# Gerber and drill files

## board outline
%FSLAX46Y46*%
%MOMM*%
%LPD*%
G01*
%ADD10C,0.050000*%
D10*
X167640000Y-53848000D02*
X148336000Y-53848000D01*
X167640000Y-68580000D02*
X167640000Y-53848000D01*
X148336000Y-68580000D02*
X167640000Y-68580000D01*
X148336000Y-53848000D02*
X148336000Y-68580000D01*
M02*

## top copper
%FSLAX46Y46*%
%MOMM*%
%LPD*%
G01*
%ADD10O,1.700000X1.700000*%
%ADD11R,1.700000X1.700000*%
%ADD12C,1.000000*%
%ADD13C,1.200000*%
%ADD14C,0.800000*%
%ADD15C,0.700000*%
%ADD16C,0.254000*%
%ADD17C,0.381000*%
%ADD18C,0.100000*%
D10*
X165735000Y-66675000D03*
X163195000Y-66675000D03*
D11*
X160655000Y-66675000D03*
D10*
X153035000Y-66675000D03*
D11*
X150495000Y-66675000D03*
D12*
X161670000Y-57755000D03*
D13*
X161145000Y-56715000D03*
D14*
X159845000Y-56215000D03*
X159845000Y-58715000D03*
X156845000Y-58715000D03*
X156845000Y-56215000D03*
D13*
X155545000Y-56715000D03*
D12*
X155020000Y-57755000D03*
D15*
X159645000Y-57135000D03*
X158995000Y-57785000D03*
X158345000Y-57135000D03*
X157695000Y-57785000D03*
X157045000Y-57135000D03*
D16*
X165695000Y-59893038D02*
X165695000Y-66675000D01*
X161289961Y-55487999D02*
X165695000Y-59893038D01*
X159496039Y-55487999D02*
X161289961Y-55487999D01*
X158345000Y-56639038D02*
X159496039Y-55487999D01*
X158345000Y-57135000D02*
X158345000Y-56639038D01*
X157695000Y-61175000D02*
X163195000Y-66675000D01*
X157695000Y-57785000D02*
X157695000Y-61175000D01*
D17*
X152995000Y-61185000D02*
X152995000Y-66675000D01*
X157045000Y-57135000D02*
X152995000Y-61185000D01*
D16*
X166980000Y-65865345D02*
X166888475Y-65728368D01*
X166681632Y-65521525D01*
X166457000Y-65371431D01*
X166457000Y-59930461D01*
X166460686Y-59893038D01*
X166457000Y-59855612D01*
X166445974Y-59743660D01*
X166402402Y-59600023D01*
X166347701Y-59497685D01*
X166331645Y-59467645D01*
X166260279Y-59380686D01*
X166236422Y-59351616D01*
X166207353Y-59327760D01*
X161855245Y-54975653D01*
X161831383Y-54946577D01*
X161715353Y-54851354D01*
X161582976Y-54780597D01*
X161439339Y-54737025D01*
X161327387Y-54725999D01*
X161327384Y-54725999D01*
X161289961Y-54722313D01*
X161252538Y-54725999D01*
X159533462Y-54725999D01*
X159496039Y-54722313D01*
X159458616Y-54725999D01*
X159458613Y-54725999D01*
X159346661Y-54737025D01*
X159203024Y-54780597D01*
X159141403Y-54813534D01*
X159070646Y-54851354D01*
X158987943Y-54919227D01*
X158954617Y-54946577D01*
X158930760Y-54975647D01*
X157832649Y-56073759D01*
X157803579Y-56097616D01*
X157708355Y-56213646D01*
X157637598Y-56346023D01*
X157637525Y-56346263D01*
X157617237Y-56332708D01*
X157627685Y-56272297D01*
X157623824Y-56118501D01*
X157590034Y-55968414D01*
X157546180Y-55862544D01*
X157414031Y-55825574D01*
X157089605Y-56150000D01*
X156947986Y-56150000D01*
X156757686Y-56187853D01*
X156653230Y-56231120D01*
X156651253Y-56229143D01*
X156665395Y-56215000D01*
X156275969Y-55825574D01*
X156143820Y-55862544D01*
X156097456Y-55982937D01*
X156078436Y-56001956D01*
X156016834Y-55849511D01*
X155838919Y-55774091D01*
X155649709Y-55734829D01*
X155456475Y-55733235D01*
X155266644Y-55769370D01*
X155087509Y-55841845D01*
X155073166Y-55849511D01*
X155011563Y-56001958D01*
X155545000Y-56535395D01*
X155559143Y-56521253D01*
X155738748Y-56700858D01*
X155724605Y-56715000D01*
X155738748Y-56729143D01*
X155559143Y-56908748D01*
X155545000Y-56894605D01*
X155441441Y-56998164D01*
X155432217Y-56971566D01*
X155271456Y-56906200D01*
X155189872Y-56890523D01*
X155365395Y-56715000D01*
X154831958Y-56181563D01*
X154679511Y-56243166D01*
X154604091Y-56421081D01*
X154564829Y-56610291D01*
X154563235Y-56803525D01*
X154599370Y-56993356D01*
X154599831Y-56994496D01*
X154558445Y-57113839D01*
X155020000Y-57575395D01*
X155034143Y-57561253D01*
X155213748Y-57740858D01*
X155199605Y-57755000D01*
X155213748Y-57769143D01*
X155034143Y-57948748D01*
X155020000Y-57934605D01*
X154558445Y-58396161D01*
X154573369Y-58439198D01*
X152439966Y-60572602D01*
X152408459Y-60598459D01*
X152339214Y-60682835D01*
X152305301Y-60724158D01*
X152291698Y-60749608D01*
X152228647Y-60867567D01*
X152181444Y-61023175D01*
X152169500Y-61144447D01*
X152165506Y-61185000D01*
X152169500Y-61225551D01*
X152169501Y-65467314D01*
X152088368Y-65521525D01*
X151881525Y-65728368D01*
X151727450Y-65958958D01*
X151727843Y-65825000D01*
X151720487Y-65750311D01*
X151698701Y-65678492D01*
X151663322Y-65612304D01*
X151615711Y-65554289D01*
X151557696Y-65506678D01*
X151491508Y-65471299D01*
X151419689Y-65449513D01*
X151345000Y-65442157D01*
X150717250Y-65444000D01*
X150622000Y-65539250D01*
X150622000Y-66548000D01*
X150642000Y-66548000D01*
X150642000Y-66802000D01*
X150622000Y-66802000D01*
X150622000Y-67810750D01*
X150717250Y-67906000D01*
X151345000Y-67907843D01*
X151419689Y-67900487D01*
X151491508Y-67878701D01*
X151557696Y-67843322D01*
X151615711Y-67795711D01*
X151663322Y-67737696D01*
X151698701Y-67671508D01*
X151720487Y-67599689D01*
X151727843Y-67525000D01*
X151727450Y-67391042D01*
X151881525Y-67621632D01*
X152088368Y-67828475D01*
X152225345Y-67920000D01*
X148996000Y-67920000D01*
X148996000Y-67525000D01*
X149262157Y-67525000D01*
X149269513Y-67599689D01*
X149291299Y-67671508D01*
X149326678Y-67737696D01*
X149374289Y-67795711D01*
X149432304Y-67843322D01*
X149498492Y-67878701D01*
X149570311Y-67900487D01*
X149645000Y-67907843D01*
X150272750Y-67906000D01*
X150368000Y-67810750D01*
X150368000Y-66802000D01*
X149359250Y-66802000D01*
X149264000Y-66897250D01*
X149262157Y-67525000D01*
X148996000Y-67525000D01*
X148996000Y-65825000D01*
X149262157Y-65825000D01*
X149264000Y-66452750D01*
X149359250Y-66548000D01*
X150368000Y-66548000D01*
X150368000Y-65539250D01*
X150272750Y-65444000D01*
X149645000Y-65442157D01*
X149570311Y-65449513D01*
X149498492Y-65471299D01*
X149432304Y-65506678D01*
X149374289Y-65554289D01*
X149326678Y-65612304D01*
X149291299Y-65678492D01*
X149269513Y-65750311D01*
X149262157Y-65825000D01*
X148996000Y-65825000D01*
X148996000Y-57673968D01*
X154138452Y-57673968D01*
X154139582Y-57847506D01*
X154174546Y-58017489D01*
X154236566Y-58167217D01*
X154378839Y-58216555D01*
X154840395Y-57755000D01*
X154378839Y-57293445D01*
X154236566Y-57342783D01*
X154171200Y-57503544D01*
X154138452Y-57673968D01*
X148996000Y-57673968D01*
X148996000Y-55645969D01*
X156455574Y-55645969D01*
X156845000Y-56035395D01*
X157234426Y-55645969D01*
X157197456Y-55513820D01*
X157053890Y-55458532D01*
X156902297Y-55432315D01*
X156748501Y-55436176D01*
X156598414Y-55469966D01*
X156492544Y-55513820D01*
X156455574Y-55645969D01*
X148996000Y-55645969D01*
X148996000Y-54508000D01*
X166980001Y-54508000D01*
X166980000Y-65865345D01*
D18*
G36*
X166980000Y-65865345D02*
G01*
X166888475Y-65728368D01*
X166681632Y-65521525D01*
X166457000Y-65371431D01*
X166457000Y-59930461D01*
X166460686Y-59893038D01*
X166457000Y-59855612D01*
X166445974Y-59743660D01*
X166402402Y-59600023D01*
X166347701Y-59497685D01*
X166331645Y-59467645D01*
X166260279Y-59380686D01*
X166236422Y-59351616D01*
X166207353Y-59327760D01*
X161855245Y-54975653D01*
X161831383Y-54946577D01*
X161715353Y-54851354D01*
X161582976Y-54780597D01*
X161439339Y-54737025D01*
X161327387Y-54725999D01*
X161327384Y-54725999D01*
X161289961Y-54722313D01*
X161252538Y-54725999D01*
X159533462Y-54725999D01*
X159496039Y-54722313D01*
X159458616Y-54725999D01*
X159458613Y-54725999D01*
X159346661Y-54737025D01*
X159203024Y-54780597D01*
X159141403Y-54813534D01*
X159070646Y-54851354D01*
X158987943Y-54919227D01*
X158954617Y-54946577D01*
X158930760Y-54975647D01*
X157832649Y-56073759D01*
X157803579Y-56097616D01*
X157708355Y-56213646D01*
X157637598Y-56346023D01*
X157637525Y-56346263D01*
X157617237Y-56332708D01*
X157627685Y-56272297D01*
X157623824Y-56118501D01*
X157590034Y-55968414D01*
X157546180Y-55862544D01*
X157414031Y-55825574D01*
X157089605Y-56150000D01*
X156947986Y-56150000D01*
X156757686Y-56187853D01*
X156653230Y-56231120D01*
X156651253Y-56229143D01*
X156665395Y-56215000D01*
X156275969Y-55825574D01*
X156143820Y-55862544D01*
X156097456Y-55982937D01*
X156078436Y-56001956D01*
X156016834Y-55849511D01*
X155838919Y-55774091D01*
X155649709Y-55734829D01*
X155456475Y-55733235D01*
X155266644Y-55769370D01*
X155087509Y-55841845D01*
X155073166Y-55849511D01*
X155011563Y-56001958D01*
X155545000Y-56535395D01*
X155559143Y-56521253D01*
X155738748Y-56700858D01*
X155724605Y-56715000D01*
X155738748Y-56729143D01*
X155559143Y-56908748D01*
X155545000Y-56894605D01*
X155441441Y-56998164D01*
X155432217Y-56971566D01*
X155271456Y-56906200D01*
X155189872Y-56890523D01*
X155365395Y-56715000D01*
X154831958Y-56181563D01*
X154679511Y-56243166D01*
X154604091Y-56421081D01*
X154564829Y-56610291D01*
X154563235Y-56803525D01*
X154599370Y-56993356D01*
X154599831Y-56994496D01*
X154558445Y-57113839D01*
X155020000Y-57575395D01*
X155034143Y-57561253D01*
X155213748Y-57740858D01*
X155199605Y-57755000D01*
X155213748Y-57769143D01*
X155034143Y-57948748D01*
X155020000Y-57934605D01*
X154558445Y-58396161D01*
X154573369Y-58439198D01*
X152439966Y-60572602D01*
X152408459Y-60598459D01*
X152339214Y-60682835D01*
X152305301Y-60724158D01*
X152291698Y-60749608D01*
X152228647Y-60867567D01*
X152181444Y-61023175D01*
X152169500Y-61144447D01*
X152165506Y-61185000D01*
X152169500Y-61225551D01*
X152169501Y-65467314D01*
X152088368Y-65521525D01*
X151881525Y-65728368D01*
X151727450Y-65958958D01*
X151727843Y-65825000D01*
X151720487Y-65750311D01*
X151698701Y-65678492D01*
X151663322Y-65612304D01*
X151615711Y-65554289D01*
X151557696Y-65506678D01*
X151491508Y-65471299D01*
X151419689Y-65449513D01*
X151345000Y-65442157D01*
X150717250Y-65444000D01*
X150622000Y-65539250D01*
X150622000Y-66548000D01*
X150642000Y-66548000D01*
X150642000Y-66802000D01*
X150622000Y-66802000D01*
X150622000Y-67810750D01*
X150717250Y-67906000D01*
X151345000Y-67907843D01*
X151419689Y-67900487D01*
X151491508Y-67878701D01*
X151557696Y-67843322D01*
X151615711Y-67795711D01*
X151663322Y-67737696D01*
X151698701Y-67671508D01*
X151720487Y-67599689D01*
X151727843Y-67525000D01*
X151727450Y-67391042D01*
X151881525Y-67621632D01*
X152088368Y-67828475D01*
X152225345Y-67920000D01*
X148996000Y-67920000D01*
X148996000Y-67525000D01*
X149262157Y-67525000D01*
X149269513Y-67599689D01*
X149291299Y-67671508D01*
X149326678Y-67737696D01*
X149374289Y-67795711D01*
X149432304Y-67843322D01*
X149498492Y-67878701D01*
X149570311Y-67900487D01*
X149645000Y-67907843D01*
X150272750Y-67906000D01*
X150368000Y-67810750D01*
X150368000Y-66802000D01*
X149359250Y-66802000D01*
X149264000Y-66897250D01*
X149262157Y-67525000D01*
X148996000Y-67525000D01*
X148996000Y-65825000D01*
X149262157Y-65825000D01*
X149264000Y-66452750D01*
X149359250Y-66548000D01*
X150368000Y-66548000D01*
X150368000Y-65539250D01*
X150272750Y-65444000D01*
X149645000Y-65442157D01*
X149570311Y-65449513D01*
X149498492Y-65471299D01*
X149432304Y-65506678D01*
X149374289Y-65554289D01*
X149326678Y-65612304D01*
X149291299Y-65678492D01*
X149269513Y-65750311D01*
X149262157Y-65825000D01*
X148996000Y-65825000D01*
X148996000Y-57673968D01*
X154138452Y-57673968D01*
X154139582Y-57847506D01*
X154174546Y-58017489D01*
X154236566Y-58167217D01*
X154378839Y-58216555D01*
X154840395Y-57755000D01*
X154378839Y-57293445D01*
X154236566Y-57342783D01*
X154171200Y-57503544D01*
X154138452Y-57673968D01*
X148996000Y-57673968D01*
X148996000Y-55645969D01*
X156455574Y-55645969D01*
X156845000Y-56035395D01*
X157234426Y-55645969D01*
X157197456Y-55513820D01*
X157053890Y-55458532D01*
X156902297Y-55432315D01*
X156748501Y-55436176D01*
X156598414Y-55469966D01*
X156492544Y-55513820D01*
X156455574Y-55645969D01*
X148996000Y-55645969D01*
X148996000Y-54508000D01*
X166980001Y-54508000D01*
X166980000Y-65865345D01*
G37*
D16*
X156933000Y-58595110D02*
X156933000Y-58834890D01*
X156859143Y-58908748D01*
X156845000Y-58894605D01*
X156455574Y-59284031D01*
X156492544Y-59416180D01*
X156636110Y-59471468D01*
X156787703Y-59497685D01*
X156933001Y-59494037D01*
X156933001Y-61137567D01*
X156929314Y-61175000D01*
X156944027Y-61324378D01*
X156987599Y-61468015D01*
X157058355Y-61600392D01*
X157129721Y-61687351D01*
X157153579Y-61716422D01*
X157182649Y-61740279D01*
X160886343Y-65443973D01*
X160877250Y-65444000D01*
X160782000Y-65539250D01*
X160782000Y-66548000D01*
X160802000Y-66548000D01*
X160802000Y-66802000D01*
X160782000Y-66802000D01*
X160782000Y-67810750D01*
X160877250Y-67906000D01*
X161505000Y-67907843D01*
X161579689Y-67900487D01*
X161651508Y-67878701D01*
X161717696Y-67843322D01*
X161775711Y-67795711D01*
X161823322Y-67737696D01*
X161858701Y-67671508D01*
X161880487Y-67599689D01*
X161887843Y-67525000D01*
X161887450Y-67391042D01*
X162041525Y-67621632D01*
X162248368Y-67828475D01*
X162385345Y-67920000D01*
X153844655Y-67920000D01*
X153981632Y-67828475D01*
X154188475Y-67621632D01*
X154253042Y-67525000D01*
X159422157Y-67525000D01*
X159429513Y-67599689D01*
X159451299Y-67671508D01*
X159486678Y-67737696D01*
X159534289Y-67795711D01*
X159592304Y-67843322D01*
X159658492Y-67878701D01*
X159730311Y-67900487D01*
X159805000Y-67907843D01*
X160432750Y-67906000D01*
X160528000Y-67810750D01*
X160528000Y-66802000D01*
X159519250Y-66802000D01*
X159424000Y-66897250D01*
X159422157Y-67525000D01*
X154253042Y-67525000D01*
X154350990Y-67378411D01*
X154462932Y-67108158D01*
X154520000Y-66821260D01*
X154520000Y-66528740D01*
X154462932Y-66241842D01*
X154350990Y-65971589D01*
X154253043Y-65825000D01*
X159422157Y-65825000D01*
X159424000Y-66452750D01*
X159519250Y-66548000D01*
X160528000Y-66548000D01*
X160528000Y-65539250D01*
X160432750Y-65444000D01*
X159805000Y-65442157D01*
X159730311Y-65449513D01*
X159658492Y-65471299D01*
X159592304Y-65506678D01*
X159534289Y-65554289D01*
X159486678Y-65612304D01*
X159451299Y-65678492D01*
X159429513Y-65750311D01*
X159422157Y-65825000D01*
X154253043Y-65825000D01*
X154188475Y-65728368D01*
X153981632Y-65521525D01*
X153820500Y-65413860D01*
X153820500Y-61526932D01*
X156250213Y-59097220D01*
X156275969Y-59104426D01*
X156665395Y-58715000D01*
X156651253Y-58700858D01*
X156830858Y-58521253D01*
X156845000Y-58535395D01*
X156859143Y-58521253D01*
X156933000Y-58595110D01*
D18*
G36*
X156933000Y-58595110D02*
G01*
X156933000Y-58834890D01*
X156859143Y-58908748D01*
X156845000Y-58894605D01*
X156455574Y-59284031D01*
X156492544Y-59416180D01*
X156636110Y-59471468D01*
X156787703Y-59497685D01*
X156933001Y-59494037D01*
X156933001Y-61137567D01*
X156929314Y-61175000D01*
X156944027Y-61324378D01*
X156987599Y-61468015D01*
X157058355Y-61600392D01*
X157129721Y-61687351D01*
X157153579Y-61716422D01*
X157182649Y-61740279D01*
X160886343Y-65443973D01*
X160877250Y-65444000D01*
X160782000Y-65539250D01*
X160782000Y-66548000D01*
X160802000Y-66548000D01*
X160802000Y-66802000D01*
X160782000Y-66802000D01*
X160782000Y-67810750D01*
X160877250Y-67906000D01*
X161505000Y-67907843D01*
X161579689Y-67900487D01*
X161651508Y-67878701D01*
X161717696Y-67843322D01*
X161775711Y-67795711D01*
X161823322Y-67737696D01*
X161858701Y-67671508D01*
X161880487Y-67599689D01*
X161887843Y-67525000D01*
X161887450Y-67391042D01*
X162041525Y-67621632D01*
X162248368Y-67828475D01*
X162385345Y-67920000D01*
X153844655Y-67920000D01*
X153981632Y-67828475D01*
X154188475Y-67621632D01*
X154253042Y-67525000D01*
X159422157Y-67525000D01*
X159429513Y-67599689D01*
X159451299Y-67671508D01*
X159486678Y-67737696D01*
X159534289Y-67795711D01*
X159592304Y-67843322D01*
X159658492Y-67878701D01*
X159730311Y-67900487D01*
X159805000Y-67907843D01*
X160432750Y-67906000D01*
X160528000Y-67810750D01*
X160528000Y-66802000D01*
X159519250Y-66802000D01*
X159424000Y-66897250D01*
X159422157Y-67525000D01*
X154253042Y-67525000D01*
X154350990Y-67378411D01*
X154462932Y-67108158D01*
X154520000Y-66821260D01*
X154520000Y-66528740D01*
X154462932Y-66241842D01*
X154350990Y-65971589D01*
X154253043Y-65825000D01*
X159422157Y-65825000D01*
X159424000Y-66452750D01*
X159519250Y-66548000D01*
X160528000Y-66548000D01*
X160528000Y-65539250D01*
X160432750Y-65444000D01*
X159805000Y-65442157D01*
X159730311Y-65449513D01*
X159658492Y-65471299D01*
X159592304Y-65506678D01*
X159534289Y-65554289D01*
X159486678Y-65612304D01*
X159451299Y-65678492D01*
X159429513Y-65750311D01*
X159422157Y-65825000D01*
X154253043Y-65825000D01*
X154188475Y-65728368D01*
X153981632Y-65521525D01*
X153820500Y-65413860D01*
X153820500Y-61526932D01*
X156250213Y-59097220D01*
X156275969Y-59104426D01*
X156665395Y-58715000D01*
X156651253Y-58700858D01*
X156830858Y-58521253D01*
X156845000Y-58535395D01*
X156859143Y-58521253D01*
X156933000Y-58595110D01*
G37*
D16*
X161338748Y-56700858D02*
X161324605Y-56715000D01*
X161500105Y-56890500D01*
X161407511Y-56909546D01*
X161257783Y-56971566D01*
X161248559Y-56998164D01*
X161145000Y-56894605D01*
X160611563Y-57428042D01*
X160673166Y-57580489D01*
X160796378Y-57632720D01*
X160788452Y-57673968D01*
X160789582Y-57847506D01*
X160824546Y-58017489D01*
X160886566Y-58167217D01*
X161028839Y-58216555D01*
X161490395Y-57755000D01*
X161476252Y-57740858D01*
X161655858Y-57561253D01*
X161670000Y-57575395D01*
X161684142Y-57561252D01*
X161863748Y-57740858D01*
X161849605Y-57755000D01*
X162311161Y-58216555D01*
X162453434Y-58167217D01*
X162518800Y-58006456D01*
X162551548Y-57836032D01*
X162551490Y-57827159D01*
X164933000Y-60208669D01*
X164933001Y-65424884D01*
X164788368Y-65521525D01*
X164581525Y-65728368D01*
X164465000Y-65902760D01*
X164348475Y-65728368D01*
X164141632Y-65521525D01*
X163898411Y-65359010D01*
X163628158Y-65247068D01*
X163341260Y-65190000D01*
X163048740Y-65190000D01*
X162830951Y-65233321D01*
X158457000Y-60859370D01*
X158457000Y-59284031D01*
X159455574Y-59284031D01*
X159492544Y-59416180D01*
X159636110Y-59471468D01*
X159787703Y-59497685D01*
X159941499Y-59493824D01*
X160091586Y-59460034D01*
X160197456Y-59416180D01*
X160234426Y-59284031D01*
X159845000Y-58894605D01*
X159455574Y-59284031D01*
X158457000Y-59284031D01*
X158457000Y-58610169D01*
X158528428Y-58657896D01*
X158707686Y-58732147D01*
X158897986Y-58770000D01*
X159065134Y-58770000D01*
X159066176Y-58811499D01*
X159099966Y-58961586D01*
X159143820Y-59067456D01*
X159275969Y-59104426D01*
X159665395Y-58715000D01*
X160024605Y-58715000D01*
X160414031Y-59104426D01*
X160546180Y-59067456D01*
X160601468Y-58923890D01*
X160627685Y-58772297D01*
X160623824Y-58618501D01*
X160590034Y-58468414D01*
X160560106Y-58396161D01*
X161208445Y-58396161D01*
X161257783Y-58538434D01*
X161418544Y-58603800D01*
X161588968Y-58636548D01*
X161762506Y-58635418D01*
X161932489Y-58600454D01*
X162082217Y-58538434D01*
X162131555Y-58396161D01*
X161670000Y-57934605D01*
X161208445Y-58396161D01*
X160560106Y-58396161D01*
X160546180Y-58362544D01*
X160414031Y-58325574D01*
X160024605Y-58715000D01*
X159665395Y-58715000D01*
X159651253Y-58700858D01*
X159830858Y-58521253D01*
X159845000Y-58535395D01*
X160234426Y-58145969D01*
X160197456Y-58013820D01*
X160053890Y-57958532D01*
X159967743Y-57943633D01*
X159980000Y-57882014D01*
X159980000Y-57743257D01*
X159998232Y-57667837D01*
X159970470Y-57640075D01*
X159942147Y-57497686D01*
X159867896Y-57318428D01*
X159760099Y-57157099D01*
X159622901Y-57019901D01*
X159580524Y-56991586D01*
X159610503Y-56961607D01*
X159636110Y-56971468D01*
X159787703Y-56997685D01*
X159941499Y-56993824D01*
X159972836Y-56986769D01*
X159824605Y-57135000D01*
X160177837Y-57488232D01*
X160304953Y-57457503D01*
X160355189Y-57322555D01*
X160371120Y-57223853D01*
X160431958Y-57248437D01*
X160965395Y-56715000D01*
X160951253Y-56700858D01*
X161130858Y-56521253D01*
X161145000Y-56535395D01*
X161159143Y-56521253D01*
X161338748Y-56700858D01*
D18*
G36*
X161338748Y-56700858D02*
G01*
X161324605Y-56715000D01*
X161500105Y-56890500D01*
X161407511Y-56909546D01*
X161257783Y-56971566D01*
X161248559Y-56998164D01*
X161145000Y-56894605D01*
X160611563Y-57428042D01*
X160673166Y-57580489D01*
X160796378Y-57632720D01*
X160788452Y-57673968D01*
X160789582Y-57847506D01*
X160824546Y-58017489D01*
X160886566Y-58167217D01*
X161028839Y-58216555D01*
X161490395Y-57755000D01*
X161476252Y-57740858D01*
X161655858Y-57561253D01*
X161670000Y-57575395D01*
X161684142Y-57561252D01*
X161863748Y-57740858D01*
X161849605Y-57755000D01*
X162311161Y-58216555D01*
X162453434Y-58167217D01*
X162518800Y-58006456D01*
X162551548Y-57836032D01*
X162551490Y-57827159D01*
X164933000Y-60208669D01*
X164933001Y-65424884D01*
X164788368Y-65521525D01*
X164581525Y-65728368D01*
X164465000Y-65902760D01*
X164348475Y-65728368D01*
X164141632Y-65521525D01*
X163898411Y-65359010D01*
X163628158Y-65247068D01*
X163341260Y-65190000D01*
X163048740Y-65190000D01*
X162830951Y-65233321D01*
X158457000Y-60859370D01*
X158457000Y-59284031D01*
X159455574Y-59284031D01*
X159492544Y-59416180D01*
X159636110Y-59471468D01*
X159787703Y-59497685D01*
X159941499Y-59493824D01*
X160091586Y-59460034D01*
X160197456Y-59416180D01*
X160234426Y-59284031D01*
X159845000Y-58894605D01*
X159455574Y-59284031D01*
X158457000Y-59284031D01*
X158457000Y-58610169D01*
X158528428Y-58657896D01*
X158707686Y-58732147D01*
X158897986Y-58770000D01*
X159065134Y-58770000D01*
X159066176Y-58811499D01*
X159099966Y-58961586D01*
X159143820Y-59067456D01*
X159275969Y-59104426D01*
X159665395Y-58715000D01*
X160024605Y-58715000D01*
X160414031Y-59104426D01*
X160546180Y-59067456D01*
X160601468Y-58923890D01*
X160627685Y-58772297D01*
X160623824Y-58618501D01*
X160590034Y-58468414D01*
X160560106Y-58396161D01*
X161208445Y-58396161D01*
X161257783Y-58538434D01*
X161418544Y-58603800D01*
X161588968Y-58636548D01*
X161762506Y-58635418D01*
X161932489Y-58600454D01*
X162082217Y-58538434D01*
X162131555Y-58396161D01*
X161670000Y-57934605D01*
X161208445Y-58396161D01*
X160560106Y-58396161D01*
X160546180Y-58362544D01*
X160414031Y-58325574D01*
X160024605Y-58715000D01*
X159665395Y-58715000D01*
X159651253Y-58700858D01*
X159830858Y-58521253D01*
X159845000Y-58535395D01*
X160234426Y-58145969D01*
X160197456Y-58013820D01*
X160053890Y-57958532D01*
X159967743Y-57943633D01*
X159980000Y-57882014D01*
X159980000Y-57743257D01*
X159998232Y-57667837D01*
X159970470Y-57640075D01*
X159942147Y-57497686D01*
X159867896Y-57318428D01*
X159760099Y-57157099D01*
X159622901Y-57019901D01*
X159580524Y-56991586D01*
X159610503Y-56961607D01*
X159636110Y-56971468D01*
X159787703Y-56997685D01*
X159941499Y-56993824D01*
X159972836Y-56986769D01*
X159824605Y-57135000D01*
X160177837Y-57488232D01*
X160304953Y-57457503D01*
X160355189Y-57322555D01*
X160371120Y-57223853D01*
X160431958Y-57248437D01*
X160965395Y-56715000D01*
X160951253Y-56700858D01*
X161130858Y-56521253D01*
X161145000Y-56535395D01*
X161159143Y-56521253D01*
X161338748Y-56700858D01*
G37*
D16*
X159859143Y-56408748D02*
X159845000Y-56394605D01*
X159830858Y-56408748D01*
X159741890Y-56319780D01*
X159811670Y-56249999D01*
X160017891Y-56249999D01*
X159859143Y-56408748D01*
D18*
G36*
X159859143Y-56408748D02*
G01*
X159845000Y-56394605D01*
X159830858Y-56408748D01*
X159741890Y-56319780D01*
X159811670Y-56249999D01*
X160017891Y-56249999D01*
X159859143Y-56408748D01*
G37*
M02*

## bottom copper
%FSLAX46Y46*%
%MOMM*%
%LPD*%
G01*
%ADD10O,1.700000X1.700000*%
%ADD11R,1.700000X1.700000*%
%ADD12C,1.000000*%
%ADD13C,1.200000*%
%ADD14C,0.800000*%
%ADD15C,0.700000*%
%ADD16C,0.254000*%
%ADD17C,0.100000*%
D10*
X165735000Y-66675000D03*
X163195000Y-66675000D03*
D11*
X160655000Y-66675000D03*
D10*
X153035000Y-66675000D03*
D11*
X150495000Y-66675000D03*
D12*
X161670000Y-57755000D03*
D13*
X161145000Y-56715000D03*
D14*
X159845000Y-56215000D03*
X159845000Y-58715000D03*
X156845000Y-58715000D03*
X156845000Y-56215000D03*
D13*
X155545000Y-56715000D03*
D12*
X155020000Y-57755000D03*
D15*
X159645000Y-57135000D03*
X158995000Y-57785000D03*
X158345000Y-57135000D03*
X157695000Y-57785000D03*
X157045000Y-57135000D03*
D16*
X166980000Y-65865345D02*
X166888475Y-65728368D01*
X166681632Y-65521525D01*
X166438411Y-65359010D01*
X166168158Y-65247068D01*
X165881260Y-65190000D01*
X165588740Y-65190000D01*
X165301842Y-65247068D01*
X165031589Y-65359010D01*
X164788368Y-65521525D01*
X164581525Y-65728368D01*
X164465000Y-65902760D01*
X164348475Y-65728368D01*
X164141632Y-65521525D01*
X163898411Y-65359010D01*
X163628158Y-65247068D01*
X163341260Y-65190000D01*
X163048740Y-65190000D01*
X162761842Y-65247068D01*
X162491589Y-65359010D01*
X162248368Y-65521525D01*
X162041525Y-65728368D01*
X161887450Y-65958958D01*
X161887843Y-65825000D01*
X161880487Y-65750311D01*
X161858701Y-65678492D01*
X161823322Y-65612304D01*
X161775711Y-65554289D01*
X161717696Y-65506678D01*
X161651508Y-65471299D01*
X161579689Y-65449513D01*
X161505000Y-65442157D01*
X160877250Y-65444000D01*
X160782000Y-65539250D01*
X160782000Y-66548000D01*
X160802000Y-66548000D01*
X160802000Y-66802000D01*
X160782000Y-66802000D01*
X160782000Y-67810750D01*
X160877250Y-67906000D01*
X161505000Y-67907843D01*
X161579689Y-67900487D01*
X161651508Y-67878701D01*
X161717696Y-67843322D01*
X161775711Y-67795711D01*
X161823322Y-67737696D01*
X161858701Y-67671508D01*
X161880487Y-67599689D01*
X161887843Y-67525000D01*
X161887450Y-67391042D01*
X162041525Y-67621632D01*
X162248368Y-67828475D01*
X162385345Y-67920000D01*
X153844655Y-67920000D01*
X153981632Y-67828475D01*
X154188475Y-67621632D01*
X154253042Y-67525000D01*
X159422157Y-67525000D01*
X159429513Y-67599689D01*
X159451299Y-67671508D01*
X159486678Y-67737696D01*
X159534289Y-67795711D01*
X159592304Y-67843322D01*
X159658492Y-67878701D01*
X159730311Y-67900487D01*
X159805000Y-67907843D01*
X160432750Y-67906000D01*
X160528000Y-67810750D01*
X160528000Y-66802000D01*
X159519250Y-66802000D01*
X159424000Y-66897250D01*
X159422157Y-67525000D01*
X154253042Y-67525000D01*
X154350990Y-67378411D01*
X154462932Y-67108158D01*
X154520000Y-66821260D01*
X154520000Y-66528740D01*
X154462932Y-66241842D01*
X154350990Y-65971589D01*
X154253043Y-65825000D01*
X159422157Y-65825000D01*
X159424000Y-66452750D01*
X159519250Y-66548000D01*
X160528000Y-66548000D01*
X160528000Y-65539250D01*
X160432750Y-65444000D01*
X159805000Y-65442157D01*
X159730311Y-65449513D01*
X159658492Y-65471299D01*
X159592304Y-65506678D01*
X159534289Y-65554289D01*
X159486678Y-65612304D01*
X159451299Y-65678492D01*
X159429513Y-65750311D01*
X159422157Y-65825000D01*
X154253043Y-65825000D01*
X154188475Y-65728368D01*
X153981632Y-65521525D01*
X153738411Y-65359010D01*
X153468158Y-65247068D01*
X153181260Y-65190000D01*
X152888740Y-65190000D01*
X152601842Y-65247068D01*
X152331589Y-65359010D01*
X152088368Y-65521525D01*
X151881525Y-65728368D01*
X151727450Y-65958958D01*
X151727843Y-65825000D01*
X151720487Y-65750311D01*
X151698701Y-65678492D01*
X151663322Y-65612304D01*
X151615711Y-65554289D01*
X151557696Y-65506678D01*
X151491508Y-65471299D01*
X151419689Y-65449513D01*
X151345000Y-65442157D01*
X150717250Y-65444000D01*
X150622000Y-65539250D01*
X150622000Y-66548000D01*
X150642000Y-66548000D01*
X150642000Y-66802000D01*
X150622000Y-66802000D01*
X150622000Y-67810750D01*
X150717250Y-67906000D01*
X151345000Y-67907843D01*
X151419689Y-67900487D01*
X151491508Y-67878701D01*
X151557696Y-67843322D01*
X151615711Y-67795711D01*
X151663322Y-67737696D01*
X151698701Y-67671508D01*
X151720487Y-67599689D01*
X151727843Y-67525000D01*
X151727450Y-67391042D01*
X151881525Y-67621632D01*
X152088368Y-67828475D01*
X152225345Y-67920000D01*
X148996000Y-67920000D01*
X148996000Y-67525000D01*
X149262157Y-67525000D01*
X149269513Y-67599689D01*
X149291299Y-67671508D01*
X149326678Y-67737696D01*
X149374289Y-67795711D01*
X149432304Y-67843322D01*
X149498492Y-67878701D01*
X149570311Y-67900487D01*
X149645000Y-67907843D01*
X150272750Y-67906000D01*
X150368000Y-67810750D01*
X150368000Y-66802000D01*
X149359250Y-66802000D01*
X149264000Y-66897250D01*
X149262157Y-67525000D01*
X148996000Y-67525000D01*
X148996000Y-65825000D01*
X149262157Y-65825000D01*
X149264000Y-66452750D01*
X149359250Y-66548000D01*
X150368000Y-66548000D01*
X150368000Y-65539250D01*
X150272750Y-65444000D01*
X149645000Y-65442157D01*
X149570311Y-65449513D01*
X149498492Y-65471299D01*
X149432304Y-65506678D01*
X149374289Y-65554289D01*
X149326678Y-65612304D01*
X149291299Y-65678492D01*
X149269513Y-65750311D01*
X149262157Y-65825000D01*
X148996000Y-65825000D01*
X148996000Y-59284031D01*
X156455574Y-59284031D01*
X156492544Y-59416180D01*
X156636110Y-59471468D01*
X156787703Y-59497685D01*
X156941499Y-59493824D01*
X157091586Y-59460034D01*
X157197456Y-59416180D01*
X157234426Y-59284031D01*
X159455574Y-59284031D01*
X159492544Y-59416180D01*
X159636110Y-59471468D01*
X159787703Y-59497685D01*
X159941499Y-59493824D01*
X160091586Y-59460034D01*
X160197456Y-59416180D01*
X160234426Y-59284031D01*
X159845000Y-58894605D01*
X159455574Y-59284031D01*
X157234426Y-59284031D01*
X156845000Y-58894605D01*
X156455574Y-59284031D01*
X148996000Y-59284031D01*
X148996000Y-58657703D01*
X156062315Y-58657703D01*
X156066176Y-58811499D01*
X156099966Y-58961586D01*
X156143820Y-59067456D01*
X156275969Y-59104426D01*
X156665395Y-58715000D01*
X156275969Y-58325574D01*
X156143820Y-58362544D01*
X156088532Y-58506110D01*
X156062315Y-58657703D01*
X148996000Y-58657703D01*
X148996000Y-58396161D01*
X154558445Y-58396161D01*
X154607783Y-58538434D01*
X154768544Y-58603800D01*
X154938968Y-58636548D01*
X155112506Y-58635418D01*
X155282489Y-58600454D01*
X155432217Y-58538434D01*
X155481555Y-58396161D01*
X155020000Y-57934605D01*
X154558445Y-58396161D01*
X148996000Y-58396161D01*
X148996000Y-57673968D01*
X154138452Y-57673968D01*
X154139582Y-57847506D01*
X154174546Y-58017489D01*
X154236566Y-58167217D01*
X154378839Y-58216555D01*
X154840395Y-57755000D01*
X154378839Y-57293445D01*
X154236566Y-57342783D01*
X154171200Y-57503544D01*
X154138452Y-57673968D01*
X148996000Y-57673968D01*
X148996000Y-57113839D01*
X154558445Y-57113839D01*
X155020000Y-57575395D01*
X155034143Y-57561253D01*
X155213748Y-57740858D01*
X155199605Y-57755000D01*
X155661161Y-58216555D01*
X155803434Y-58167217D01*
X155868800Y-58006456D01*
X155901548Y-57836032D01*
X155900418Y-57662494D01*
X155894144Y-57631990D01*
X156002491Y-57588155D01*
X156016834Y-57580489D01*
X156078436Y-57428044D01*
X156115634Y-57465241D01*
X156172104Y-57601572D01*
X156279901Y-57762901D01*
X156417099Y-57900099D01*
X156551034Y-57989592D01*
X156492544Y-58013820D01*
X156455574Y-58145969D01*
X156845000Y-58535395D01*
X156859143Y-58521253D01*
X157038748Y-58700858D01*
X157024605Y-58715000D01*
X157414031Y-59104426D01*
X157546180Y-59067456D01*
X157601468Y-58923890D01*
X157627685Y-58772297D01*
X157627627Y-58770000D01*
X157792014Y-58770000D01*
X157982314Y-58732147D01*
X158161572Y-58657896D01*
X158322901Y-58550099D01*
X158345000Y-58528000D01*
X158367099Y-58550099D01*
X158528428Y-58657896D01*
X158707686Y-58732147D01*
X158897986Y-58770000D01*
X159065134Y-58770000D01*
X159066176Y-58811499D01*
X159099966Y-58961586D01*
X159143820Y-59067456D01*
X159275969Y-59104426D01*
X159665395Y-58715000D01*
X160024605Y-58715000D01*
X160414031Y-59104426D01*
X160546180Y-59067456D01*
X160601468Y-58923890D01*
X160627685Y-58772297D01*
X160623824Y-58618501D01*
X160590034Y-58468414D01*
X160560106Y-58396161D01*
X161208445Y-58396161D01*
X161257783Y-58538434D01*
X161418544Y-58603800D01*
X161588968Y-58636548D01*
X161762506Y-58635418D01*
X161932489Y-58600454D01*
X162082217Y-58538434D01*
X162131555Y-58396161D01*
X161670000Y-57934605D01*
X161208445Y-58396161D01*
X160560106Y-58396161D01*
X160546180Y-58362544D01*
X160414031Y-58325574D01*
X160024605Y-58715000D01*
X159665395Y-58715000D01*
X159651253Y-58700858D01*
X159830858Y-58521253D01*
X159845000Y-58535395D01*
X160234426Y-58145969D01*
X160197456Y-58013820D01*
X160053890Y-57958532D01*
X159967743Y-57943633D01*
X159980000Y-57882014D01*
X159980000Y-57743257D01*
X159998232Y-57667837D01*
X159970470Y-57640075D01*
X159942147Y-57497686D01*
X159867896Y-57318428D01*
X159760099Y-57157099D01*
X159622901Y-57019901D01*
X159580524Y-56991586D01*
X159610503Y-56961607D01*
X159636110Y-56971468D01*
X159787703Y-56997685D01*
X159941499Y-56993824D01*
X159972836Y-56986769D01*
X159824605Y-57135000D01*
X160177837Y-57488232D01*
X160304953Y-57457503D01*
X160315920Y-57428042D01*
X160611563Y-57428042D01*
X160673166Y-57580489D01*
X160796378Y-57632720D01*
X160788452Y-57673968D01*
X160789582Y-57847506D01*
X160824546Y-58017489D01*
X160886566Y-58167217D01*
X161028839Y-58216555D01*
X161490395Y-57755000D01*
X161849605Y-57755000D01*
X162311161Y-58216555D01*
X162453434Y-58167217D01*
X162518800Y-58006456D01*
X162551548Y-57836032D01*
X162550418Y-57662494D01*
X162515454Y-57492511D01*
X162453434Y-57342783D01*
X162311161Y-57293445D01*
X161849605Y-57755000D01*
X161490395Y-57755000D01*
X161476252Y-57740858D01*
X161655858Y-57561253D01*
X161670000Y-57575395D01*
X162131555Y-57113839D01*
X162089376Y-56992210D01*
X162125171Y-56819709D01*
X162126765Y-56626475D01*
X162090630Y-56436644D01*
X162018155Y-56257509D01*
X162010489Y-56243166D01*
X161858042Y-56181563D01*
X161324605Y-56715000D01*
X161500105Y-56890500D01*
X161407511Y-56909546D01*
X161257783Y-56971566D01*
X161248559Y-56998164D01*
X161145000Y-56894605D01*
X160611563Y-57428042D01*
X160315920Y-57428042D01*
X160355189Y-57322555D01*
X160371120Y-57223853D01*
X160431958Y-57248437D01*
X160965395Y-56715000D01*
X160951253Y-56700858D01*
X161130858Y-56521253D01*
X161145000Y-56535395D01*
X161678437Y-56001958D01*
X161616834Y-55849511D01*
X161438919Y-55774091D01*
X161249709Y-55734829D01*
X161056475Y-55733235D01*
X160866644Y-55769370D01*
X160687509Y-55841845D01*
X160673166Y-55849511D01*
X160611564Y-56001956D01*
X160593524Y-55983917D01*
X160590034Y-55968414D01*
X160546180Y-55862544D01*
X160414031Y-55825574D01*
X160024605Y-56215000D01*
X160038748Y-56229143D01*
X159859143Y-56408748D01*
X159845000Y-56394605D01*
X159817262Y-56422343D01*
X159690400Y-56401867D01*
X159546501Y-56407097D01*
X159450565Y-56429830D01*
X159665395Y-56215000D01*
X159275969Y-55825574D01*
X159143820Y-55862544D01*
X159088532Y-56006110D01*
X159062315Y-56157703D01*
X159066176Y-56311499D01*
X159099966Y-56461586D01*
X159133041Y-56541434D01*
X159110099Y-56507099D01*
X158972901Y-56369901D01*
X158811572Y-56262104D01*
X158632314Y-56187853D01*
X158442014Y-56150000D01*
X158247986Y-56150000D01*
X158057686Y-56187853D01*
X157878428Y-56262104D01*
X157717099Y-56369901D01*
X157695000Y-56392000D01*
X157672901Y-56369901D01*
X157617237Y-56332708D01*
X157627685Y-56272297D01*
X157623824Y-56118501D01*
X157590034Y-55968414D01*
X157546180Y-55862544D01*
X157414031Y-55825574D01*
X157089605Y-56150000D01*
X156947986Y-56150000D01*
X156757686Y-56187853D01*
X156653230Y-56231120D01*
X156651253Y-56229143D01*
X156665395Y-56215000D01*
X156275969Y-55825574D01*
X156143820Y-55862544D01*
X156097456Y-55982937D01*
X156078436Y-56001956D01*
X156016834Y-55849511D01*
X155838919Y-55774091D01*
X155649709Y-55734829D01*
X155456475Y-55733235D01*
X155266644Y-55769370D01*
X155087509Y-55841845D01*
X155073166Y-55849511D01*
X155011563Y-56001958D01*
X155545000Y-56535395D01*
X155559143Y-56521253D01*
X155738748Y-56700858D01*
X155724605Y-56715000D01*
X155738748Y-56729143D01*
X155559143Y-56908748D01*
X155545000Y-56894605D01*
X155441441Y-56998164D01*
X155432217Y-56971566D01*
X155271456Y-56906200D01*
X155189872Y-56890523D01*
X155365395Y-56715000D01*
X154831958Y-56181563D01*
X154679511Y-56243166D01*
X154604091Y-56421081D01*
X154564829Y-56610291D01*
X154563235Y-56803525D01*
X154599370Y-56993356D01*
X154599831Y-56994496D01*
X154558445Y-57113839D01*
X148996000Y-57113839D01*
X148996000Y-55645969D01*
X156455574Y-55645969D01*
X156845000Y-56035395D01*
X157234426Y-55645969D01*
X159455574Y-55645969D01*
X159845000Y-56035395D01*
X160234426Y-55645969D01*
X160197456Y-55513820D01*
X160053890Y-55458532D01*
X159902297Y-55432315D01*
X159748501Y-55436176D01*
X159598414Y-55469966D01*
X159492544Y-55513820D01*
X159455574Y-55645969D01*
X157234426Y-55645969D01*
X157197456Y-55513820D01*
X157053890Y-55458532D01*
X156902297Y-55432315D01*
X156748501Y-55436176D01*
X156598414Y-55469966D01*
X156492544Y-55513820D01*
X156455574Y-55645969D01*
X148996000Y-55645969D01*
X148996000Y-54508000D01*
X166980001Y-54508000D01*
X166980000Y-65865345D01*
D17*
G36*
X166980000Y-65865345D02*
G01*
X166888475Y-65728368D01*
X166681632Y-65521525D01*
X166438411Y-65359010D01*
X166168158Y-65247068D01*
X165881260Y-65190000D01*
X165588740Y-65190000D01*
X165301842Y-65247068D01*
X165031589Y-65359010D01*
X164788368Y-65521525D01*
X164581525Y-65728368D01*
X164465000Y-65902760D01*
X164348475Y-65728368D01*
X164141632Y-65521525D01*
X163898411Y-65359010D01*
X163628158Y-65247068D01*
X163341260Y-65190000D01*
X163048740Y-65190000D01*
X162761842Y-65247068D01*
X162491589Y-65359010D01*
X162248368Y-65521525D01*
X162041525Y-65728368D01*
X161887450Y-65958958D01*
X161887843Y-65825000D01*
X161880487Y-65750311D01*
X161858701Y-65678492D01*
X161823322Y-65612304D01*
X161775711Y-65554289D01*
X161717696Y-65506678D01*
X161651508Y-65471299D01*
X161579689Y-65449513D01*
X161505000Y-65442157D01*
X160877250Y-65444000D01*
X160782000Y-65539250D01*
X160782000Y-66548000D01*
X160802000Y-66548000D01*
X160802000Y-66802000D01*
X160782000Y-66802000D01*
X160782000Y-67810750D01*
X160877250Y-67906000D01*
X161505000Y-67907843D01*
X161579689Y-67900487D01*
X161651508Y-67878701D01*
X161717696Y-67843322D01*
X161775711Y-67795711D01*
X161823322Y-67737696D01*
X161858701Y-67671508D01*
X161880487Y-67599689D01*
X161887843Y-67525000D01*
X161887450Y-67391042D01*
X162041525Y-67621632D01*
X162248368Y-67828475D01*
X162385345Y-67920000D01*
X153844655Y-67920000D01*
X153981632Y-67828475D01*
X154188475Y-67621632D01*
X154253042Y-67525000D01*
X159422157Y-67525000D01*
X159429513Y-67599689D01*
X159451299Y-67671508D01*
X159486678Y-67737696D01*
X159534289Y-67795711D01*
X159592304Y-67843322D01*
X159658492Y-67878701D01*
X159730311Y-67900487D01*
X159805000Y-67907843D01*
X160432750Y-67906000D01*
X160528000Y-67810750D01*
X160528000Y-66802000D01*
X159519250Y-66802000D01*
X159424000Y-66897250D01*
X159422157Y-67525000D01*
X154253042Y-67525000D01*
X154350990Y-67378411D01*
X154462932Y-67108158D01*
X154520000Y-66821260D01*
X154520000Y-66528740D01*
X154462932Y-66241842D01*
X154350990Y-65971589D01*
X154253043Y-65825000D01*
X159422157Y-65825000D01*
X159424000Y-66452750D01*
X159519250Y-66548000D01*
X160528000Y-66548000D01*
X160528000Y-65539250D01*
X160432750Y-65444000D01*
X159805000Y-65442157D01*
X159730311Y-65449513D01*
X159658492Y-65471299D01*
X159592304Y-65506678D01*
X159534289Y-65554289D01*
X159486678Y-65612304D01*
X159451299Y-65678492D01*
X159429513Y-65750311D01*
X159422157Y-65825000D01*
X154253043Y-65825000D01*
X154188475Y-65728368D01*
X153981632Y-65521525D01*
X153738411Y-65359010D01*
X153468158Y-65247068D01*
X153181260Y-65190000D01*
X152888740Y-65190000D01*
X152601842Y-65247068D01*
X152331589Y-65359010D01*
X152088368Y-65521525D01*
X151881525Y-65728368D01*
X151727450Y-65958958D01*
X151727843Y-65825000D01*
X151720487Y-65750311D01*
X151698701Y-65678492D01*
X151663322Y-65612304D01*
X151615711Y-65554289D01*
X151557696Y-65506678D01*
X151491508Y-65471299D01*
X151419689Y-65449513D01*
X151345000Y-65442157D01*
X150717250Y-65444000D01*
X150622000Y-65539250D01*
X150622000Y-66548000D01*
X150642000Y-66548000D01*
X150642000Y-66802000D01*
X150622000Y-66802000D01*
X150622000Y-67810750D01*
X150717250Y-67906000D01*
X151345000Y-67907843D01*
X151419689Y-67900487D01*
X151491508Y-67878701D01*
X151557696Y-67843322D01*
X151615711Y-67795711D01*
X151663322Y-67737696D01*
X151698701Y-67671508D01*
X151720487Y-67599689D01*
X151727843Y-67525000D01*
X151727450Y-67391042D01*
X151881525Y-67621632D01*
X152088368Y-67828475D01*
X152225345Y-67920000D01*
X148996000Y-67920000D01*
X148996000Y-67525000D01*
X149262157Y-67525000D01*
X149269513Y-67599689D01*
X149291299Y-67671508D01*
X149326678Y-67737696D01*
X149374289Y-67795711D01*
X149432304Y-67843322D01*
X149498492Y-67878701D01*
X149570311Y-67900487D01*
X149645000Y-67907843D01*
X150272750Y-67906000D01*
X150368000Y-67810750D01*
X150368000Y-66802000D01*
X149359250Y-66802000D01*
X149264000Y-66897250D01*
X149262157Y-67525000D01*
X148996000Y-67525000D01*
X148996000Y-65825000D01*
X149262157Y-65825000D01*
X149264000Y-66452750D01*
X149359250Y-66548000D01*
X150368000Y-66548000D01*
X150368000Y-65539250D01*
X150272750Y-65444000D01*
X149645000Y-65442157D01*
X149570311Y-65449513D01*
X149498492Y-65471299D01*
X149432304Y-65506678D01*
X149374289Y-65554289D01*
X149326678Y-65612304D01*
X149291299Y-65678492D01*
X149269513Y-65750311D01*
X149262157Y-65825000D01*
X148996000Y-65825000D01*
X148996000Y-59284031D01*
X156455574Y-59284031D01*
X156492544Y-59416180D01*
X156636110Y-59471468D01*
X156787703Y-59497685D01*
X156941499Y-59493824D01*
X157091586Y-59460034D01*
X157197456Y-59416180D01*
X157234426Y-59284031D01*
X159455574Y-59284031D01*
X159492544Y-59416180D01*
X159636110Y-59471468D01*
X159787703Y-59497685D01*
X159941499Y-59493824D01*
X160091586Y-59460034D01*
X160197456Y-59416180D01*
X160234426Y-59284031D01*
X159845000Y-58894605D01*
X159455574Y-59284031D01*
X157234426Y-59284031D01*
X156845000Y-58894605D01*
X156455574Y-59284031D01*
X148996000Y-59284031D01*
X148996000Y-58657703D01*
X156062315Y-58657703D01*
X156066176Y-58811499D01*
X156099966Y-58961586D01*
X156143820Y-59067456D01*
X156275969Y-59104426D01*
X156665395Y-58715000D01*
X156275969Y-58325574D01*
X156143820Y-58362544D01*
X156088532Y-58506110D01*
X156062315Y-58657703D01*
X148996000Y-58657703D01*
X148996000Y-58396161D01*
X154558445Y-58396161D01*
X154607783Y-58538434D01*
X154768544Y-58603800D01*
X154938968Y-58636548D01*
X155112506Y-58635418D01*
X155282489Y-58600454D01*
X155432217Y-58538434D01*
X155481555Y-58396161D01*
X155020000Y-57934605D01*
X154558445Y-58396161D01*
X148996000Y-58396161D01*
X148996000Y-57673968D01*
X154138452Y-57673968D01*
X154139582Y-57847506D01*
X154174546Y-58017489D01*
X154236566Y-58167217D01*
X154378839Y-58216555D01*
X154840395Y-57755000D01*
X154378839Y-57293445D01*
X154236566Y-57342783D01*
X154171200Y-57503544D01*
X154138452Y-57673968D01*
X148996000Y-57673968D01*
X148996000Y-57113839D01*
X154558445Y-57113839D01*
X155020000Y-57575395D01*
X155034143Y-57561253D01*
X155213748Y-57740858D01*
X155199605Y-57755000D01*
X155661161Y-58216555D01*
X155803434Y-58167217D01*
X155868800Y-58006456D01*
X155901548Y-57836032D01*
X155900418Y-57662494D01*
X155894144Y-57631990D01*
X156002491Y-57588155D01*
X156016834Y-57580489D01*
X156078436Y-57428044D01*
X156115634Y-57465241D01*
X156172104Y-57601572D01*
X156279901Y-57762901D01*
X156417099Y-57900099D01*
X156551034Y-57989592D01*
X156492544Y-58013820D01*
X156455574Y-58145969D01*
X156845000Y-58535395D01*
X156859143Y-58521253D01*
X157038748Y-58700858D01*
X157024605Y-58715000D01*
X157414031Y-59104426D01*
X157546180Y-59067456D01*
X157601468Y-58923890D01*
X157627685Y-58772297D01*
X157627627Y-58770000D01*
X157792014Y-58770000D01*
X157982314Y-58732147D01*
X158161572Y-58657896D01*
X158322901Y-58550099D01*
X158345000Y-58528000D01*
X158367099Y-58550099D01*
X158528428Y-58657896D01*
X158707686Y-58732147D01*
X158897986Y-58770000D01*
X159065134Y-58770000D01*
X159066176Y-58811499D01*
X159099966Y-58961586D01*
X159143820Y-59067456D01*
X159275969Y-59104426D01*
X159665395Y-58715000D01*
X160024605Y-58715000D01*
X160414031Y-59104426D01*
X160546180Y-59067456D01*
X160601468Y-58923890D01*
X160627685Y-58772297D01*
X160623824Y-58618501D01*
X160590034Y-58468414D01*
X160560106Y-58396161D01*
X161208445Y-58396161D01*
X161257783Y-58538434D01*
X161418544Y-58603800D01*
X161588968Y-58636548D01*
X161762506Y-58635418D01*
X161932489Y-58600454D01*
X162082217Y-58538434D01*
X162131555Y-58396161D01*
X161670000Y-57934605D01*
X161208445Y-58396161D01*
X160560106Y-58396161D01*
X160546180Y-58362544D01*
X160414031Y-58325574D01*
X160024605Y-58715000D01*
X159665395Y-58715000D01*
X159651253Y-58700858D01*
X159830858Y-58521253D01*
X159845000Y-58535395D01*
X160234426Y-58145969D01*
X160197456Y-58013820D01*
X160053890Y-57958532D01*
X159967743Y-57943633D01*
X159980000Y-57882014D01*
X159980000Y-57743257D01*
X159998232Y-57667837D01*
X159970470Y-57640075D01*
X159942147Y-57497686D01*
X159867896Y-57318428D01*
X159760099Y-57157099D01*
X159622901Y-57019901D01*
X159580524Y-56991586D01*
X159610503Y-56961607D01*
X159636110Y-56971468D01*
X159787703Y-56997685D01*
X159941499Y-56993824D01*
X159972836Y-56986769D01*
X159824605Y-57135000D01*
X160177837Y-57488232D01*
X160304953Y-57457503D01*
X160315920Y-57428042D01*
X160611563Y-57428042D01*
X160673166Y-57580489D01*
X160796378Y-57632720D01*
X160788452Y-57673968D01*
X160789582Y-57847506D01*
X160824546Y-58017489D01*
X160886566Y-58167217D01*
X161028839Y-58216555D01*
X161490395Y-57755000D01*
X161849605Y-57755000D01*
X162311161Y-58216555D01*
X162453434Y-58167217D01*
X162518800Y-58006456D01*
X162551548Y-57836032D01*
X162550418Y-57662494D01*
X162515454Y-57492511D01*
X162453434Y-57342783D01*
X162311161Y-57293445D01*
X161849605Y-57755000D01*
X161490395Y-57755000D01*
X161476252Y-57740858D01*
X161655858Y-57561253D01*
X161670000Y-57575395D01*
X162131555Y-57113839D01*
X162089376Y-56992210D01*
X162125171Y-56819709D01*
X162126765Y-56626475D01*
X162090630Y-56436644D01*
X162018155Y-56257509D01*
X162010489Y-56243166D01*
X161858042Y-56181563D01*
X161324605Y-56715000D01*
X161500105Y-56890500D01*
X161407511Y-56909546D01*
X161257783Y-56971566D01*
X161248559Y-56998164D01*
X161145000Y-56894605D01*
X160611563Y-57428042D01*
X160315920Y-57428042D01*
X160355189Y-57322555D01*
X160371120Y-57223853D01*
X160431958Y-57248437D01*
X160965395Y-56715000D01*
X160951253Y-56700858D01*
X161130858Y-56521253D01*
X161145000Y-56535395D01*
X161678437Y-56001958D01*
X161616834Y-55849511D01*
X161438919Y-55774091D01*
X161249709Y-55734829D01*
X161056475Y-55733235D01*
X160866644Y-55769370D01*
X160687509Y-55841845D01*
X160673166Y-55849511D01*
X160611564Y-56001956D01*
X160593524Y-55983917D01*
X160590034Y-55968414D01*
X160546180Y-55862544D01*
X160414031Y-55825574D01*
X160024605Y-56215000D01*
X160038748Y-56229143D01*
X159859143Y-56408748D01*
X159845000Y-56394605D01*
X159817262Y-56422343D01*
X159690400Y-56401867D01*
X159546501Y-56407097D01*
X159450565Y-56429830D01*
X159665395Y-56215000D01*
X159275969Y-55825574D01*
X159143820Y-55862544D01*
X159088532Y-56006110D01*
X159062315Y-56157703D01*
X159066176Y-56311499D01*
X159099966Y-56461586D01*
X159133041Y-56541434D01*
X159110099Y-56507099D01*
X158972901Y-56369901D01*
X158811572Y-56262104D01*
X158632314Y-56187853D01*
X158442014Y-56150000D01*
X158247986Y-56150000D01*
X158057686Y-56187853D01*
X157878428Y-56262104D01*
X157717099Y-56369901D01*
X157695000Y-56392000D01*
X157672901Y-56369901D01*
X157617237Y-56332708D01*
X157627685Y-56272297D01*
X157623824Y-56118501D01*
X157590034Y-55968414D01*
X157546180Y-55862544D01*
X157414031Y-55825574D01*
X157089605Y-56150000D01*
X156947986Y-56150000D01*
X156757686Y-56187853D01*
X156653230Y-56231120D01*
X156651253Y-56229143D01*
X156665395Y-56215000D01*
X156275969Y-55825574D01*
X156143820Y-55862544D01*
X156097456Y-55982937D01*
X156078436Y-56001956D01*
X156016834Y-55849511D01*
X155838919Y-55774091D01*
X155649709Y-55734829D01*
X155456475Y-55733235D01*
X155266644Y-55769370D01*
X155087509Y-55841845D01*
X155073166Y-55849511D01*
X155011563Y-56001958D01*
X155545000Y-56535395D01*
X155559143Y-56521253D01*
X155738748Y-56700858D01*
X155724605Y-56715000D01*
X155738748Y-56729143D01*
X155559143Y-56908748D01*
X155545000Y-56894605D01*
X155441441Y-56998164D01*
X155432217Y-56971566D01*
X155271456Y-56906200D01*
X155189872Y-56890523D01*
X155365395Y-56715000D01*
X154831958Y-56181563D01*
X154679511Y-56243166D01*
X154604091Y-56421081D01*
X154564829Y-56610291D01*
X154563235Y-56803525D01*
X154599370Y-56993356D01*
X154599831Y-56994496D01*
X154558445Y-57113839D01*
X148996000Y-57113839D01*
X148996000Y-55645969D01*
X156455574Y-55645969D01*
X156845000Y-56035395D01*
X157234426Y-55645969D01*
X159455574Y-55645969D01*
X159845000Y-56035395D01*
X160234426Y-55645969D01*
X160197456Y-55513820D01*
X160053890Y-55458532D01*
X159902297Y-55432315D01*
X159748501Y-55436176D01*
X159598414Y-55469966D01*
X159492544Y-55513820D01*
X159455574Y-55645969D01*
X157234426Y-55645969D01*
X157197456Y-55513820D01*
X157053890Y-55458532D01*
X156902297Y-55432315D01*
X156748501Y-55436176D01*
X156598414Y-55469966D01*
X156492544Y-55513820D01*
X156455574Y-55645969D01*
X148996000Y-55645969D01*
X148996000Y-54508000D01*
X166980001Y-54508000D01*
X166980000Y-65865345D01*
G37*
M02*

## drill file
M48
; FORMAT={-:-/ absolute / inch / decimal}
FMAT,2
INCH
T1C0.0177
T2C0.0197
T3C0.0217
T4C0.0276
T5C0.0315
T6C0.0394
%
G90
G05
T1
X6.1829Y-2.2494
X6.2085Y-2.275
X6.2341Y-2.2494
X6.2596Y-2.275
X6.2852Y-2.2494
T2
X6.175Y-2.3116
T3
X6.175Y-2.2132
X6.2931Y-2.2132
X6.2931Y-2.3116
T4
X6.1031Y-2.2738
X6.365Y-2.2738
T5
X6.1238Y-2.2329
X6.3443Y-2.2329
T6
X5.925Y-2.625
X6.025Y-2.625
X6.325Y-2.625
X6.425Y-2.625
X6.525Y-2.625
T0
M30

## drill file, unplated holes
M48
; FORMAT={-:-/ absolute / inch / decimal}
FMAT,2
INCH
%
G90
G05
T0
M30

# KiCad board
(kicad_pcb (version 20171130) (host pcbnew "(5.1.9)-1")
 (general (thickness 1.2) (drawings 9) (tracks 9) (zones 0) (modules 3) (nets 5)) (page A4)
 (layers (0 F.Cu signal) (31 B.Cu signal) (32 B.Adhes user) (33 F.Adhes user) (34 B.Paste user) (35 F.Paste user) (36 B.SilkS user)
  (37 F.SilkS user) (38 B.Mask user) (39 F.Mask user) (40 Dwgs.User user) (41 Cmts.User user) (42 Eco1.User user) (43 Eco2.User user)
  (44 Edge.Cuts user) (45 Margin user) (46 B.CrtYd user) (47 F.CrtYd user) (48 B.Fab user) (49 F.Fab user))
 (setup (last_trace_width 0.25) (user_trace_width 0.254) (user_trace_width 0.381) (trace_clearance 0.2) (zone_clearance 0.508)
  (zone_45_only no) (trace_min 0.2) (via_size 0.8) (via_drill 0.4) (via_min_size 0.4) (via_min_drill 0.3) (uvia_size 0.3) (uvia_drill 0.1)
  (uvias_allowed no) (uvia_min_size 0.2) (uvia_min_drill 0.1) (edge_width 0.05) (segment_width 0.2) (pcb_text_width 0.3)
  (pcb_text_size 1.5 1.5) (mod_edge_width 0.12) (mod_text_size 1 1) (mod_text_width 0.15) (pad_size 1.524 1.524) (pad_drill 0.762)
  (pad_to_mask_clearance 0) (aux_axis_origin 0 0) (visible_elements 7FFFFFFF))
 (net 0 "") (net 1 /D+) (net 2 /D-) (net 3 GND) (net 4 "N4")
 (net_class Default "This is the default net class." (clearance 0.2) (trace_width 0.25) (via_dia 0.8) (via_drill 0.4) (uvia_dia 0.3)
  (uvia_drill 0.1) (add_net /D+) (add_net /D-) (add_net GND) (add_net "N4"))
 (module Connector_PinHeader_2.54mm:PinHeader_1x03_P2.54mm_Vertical (layer F.Cu) (at 160.655 66.675 90)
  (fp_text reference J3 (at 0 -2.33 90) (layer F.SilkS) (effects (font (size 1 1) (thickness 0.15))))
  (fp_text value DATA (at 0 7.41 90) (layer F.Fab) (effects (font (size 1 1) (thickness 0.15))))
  (pad 3 thru_hole oval (at 0 5.08 90) (size 1.7 1.7) (drill 1) (layers *.Cu *.Mask) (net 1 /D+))
  (pad 2 thru_hole oval (at 0 2.54 90) (size 1.7 1.7) (drill 1) (layers *.Cu *.Mask) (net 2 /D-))
  (pad 1 thru_hole rect (at 0 0 90) (size 1.7 1.7) (drill 1) (layers *.Cu *.Mask) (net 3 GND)))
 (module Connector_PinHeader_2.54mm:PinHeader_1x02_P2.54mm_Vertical (layer F.Cu) (at 150.495 66.675 90)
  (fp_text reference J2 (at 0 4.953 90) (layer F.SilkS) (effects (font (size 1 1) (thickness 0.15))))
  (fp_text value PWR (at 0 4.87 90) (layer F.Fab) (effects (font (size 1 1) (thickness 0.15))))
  (pad 2 thru_hole oval (at 0 2.54 90) (size 1.7 1.7) (drill 1) (layers *.Cu *.Mask) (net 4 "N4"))
  (pad 1 thru_hole rect (at 0 0 90) (size 1.7 1.7) (drill 1) (layers *.Cu *.Mask) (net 3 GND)))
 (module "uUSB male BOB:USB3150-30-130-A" (layer F.Cu) (at 158.345 57.135)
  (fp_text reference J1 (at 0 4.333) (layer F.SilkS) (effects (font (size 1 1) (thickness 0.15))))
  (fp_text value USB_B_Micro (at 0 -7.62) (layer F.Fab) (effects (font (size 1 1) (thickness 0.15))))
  (pad 6 thru_hole circle (at 3.325 0.62) (size 1 1) (drill 0.7) (layers *.Cu *.Mask) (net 3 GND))
  (pad 6 thru_hole circle (at 2.8 -0.42) (size 1.2 1.2) (drill 0.8) (layers *.Cu *.Mask) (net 3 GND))
  (pad 6 thru_hole circle (at 1.5 -0.92) (size 0.8 0.8) (drill 0.55) (layers *.Cu *.Mask) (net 3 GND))
  (pad 6 thru_hole circle (at 1.5 1.58) (size 0.8 0.8) (drill 0.55) (layers *.Cu *.Mask) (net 3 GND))
  (pad 6 thru_hole circle (at -1.5 1.58) (size 0.8 0.8) (drill 0.5) (layers *.Cu *.Mask) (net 3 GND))
  (pad 6 thru_hole circle (at -1.5 -0.92) (size 0.8 0.8) (drill 0.55) (layers *.Cu *.Mask) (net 3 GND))
  (pad 6 thru_hole circle (at -2.8 -0.42) (size 1.2 1.2) (drill 0.8) (layers *.Cu *.Mask) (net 3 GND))
  (pad 6 thru_hole circle (at -3.325 0.62) (size 1 1) (drill 0.7) (layers *.Cu *.Mask) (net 3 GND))
  (pad 5 thru_hole circle (at 1.3 0) (size 0.7 0.7) (drill 0.45) (layers *.Cu *.Mask) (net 3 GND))
  (pad 4 thru_hole circle (at 0.65 0.65) (size 0.7 0.7) (drill 0.45) (layers *.Cu *.Mask))
  (pad 3 thru_hole circle (at 0 0) (size 0.7 0.7) (drill 0.45) (layers *.Cu *.Mask) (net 1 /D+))
  (pad 2 thru_hole circle (at -0.65 0.65) (size 0.7 0.7) (drill 0.45) (layers *.Cu *.Mask) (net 2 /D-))
  (pad 1 thru_hole circle (at -1.3 0) (size 0.7 0.7) (drill 0.45) (layers *.Cu *.Mask) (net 4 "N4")))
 (gr_line (start 167.64 53.848) (end 148.336 53.848) (layer Edge.Cuts) (width 0.05))
 (gr_line (start 167.64 68.58) (end 167.64 53.848) (layer Edge.Cuts) (width 0.05))
 (gr_line (start 148.336 68.58) (end 167.64 68.58) (layer Edge.Cuts) (width 0.05))
 (gr_line (start 148.336 53.848) (end 148.336 68.58) (layer Edge.Cuts) (width 0.05))
 (segment (start 165.695 59.893038) (end 165.695 66.675) (width 0.254) (layer F.Cu) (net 1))
 (segment (start 161.289961 55.487999) (end 165.695 59.893038) (width 0.254) (layer F.Cu) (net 1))
 (segment (start 159.496039 55.487999) (end 161.289961 55.487999) (width 0.254) (layer F.Cu) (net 1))
 (segment (start 158.345 56.639038) (end 159.496039 55.487999) (width 0.254) (layer F.Cu) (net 1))
 (segment (start 158.345 57.135) (end 158.345 56.639038) (width 0.254) (layer F.Cu) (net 1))
 (segment (start 157.695 61.175) (end 163.195 66.675) (width 0.254) (layer F.Cu) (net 2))
 (segment (start 157.695 57.785) (end 157.695 61.175) (width 0.254) (layer F.Cu) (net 2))
 (segment (start 152.995 61.185) (end 152.995 66.675) (width 0.381) (layer F.Cu) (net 4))
 (segment (start 157.045 57.135) (end 152.995 61.185) (width 0.381) (layer F.Cu) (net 4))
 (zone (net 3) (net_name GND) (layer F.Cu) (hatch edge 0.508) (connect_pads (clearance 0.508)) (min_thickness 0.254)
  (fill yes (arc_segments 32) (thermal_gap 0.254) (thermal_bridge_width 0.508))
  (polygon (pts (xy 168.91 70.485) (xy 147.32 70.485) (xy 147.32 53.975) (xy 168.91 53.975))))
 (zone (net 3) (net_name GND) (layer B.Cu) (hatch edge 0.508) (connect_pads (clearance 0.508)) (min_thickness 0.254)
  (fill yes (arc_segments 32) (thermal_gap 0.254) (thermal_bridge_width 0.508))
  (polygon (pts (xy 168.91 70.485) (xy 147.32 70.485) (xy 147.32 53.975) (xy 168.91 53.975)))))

